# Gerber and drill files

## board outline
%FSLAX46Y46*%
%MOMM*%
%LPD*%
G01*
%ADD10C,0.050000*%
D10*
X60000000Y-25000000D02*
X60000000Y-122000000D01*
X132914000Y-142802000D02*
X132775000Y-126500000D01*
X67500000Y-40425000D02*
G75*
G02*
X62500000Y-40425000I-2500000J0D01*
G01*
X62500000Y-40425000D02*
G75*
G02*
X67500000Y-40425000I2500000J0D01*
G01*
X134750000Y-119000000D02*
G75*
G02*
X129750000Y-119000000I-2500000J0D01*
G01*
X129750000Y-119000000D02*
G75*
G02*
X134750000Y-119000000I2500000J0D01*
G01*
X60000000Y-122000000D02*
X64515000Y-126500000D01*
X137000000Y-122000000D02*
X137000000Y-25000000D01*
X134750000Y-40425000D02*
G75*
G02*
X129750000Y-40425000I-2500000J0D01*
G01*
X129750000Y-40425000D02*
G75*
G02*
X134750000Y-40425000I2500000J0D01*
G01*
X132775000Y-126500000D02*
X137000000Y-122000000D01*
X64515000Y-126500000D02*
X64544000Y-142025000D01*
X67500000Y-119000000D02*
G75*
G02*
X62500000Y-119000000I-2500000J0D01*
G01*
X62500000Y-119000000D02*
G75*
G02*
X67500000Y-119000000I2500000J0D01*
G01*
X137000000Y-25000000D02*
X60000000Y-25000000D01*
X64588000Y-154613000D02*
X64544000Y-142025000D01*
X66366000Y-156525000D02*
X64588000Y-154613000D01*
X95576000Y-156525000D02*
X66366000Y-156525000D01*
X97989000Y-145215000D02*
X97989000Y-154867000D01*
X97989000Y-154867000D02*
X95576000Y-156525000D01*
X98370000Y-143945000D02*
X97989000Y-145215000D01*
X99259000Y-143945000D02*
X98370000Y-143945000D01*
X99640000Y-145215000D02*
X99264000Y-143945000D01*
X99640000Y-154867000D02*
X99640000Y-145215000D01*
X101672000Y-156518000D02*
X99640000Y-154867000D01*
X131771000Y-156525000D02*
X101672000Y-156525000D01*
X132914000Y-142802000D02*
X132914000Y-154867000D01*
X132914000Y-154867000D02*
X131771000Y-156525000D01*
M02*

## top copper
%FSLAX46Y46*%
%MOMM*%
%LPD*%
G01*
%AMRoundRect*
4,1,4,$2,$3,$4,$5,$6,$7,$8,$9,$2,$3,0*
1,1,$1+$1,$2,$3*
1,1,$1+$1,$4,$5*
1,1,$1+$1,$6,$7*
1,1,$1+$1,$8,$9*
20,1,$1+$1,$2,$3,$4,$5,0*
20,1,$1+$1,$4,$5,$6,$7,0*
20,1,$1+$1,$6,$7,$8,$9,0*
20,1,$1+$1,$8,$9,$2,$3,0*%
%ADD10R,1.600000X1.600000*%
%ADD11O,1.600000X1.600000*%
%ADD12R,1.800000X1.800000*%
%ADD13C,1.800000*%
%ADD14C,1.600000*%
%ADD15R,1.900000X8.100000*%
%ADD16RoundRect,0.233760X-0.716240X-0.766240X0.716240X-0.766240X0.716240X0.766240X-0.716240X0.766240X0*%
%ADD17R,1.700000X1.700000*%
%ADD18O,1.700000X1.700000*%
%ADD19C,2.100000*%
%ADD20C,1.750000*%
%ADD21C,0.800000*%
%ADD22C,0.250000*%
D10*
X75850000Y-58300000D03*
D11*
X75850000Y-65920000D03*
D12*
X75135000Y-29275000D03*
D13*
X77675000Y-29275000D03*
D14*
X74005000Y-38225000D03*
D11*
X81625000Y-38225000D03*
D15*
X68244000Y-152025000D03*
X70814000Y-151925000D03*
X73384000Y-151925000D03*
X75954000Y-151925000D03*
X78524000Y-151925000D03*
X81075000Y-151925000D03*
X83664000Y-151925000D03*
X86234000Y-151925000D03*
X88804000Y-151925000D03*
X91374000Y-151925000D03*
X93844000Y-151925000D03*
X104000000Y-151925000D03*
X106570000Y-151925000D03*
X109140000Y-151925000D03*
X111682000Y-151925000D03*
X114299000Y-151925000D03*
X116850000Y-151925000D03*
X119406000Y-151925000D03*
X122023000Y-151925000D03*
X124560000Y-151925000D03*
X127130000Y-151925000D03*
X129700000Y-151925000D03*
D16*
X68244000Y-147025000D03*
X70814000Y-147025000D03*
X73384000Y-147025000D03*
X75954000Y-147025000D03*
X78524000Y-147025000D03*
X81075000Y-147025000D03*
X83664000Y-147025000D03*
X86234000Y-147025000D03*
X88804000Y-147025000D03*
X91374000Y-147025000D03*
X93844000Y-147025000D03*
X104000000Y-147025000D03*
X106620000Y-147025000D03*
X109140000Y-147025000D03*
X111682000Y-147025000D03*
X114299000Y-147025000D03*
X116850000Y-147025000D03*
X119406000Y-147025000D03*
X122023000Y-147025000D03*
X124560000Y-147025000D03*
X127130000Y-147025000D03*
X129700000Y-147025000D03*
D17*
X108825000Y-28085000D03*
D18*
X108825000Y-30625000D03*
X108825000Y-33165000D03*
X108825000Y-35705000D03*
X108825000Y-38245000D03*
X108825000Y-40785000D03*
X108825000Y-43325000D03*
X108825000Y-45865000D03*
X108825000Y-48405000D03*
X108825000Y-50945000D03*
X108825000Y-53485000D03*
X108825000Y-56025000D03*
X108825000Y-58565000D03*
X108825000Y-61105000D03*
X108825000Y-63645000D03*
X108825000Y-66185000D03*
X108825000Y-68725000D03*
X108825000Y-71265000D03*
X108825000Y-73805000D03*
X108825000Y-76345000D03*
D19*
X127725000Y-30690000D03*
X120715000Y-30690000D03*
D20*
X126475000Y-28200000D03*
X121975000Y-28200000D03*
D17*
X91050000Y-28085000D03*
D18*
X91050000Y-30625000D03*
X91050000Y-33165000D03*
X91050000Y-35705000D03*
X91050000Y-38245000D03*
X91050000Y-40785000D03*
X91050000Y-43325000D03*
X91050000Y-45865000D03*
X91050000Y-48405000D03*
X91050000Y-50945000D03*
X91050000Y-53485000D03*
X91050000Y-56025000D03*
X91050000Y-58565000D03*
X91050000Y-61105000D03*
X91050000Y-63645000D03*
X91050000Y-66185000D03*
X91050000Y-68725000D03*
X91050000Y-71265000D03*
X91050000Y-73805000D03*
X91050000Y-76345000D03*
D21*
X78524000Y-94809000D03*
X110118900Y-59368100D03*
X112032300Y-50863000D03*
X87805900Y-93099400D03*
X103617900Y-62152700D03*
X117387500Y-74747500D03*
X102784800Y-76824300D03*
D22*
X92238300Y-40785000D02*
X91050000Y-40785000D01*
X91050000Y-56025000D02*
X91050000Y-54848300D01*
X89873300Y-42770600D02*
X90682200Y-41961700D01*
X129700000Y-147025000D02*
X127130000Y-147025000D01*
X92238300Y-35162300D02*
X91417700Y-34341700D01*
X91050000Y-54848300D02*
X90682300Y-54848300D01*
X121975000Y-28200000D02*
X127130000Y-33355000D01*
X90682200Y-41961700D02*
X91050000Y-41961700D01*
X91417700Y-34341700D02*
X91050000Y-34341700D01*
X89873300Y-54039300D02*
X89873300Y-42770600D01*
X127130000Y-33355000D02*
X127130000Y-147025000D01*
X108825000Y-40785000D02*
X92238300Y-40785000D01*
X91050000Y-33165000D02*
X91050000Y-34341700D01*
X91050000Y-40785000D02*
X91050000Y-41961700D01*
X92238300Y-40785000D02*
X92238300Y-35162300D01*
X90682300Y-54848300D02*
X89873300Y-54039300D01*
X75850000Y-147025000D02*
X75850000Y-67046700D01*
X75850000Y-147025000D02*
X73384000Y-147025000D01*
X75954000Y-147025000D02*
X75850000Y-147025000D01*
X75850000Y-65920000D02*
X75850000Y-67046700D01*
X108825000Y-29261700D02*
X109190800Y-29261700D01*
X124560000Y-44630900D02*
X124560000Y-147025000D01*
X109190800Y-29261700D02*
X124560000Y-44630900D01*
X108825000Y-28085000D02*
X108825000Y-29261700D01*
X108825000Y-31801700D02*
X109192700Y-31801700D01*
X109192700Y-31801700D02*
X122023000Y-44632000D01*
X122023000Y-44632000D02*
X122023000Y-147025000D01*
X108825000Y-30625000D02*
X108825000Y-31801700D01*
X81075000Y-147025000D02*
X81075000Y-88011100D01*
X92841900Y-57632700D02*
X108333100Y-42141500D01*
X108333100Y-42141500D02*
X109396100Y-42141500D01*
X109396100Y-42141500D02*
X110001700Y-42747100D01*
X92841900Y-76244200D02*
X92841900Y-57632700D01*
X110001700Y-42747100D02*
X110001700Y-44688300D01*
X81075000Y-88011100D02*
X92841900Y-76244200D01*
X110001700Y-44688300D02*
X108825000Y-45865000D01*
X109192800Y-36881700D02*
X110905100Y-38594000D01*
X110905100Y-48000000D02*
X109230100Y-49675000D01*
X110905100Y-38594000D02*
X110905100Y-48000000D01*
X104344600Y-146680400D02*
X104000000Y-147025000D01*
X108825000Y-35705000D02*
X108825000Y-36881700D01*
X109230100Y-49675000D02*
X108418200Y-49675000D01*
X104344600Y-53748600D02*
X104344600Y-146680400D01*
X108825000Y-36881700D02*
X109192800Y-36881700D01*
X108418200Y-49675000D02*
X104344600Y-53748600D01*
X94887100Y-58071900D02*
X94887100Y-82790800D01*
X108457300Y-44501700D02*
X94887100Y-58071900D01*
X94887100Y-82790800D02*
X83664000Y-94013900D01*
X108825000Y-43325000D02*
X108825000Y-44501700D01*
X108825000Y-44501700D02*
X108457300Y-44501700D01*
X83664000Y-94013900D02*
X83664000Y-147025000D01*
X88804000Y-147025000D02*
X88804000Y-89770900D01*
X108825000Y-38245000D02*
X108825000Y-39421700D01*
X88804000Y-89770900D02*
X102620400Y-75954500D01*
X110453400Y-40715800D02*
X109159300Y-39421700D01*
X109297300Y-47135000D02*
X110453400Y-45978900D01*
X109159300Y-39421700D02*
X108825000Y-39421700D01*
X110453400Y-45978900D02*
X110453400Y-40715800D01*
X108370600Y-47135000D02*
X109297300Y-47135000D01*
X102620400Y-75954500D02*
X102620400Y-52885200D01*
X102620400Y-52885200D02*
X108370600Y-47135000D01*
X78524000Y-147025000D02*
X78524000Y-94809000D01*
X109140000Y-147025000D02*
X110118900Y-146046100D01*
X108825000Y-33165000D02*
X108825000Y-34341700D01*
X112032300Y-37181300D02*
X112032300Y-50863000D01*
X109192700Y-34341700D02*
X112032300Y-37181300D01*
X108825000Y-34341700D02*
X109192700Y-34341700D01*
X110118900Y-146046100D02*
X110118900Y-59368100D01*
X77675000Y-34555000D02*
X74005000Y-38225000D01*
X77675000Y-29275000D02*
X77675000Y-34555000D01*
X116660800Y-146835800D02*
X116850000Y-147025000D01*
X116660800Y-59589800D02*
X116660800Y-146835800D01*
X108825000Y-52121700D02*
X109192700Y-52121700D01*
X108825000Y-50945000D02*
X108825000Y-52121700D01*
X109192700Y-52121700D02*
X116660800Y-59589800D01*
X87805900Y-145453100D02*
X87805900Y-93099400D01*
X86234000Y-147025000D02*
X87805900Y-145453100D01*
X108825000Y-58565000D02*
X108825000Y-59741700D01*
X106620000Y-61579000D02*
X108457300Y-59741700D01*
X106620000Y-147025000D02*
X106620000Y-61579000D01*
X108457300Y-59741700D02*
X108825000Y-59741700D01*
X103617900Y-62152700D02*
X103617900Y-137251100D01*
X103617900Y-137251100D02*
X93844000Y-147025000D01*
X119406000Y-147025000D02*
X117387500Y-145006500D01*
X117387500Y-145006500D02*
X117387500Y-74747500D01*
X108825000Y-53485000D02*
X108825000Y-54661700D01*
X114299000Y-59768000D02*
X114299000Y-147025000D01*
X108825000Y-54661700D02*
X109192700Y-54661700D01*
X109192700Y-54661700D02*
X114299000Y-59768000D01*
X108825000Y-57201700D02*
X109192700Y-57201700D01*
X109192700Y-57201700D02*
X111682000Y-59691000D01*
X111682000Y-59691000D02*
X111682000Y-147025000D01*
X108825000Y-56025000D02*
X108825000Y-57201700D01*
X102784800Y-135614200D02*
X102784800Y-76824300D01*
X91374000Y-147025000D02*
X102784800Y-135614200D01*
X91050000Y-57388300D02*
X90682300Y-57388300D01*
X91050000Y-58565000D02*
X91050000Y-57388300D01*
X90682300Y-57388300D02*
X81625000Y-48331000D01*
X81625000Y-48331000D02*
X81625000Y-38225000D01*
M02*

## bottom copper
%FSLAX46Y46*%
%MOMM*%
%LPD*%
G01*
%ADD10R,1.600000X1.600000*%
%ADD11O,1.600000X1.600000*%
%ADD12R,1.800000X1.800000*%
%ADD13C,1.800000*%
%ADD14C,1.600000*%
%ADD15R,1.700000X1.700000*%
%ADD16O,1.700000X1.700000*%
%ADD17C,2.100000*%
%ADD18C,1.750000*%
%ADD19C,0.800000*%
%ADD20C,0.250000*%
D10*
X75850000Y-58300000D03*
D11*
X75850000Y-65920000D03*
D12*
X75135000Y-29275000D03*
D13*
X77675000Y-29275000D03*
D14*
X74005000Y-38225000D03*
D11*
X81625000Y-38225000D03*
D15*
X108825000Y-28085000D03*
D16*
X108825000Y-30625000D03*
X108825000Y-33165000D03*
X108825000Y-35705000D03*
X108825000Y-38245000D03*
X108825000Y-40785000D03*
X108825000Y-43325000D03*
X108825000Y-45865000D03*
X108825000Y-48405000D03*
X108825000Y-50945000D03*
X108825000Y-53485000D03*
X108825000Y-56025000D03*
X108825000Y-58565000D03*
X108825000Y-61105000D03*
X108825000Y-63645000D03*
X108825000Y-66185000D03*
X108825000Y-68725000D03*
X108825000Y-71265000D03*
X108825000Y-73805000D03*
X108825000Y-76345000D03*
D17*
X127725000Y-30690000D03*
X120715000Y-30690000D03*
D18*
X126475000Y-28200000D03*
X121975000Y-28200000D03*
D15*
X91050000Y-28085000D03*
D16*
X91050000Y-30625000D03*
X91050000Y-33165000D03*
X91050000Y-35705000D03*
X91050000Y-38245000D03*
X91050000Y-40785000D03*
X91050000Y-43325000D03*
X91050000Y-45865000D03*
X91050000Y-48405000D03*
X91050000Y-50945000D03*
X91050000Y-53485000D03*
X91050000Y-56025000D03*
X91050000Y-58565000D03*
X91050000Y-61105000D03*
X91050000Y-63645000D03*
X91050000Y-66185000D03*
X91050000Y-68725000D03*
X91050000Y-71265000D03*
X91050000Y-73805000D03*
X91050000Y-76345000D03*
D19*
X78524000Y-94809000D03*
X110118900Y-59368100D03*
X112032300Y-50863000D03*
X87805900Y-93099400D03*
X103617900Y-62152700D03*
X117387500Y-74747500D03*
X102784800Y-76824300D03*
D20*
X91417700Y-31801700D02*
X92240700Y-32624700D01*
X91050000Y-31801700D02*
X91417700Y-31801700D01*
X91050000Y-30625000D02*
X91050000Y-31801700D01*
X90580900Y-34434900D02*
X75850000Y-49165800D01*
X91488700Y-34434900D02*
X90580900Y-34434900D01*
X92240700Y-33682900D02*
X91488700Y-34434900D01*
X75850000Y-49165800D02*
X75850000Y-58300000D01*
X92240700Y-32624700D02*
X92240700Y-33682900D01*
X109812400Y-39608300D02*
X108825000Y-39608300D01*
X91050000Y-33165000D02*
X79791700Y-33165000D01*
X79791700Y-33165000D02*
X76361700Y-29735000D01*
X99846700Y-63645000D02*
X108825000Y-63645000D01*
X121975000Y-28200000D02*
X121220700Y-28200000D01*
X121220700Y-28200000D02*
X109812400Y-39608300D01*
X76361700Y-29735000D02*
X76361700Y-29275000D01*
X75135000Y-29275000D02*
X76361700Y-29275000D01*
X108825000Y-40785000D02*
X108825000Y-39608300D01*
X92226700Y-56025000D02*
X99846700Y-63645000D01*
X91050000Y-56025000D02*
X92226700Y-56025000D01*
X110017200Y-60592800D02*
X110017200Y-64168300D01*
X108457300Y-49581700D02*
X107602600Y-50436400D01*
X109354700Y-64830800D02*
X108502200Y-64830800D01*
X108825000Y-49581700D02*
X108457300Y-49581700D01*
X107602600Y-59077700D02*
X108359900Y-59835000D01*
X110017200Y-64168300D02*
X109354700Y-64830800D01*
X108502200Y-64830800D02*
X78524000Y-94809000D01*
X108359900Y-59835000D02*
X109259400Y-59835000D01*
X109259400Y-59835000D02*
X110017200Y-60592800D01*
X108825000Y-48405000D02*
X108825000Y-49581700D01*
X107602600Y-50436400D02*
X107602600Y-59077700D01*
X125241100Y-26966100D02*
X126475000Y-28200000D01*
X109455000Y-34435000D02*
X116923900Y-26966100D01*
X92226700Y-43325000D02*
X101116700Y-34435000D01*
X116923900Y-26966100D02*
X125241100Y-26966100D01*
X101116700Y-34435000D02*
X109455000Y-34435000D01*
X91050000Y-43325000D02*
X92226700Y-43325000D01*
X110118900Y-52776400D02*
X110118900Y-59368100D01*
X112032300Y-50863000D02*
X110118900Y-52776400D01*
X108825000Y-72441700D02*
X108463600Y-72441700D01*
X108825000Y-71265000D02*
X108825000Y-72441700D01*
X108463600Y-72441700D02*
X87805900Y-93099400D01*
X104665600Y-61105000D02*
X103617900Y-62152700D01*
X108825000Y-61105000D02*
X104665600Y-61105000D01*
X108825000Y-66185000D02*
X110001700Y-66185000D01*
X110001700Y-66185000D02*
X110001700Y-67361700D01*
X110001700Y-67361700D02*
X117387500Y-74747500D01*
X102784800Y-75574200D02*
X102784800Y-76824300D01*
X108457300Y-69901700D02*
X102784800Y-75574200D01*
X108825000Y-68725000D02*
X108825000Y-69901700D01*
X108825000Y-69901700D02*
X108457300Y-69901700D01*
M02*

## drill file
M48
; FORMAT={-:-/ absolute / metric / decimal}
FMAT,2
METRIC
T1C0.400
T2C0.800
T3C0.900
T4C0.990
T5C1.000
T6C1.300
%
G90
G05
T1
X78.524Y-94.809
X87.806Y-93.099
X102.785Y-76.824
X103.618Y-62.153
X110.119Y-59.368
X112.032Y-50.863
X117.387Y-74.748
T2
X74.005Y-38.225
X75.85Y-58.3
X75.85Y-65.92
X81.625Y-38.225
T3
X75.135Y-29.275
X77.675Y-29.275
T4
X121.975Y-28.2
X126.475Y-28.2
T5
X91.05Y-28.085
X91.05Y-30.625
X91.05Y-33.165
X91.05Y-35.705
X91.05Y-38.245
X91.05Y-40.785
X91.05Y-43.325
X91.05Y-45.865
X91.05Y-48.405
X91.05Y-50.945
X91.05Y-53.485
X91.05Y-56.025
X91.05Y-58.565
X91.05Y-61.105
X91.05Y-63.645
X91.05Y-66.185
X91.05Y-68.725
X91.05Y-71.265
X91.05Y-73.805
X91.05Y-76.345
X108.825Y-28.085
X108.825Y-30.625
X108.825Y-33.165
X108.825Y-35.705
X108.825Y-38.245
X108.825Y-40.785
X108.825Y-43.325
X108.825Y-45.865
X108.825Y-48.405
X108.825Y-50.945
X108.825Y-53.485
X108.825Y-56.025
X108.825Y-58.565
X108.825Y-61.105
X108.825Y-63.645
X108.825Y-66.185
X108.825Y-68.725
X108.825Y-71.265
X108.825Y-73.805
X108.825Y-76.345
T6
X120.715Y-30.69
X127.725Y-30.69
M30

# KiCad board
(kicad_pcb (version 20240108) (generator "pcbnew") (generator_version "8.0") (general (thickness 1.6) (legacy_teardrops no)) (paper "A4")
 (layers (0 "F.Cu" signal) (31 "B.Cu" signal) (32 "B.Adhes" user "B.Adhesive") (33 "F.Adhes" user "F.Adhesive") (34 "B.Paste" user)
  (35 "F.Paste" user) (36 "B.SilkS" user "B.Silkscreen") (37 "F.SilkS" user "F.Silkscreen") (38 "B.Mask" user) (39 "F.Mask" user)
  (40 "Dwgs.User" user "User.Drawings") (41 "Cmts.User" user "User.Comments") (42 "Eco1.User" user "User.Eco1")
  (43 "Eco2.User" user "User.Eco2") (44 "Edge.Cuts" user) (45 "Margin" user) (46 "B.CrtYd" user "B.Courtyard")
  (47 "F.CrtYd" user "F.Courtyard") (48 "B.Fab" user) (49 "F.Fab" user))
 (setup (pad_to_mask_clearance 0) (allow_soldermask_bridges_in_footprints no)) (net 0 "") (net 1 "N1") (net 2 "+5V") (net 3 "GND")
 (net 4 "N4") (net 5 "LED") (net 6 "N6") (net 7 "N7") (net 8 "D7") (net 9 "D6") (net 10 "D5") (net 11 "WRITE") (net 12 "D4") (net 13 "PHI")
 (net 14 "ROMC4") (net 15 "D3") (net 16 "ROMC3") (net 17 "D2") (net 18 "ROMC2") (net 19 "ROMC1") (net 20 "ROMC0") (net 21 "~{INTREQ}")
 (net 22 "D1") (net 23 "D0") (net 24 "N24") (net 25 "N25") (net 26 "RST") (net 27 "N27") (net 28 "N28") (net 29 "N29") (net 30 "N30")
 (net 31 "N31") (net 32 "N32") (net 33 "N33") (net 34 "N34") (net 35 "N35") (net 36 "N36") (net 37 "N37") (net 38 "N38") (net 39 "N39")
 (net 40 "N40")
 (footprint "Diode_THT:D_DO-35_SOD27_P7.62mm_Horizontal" (layer "F.Cu") (at 75.85 58.3 -90)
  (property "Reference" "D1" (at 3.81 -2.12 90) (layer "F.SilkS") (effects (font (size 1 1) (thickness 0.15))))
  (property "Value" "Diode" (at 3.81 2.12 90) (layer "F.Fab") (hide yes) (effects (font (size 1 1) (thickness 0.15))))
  (pad "1" thru_hole rect (at 0 0 270) (size 1.6 1.6) (drill 0.8) (layers "*.Cu" "*.Mask") (remove_unused_layers no) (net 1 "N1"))
  (pad "2" thru_hole oval (at 7.62 0 270) (size 1.6 1.6) (drill 0.8) (layers "*.Cu" "*.Mask") (remove_unused_layers no) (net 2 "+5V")))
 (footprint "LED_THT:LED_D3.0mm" (layer "F.Cu") (at 75.135 29.275)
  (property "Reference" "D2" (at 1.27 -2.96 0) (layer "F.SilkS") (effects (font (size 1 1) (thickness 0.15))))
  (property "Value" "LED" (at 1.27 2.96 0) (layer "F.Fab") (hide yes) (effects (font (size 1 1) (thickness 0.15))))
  (pad "1" thru_hole rect (at 0 0) (size 1.8 1.8) (drill 0.9) (layers "*.Cu" "*.Mask") (remove_unused_layers no) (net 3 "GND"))
  (pad "2" thru_hole circle (at 2.54 0) (size 1.8 1.8) (drill 0.9) (layers "*.Cu" "*.Mask") (remove_unused_layers no) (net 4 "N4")))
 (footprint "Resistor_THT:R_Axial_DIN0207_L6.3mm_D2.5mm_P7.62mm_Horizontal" (layer "F.Cu") (at 74.005 38.225)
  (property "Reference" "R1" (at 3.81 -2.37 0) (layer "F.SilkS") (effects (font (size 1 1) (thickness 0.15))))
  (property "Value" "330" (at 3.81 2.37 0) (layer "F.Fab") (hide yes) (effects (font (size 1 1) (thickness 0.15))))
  (pad "1" thru_hole circle (at 0 0) (size 1.6 1.6) (drill 0.8) (layers "*.Cu" "*.Mask") (remove_unused_layers no) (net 4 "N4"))
  (pad "2" thru_hole oval (at 7.62 0) (size 1.6 1.6) (drill 0.8) (layers "*.Cu" "*.Mask") (remove_unused_layers no) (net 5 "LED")))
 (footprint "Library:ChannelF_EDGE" (layer "F.Cu") (at 68.144 149.025)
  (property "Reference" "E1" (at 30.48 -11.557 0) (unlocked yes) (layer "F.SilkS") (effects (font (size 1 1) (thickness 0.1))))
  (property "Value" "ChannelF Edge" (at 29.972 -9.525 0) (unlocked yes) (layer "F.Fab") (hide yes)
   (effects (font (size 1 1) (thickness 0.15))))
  (fp_line (start -3.556 5.588) (end -3.6 -7) (stroke (width 0.05) (type default)) (layer "Edge.Cuts"))
  (fp_line (start -1.778 7.5) (end -3.556 5.588) (stroke (width 0.05) (type default)) (layer "Edge.Cuts"))
  (fp_line (start 27.432 7.5) (end -1.778 7.5) (stroke (width 0.05) (type default)) (layer "Edge.Cuts"))
  (fp_line (start 29.845 -3.81) (end 29.845 5.842) (stroke (width 0.05) (type default)) (layer "Edge.Cuts"))
  (fp_line (start 29.845 5.842) (end 27.432 7.5) (stroke (width 0.05) (type default)) (layer "Edge.Cuts"))
  (fp_line (start 30.226 -5.08) (end 29.845 -3.81) (stroke (width 0.05) (type default)) (layer "Edge.Cuts"))
  (fp_line (start 31.115 -5.08) (end 30.226 -5.08) (stroke (width 0.05) (type default)) (layer "Edge.Cuts"))
  (fp_line (start 31.496 -3.81) (end 31.12 -5.08) (stroke (width 0.05) (type default)) (layer "Edge.Cuts"))
  (fp_line (start 31.496 5.842) (end 31.496 -3.81) (stroke (width 0.05) (type default)) (layer "Edge.Cuts"))
  (fp_line (start 33.528 7.493) (end 31.496 5.842) (stroke (width 0.05) (type default)) (layer "Edge.Cuts"))
  (fp_line (start 63.627 7.5) (end 33.528 7.5) (stroke (width 0.05) (type default)) (layer "Edge.Cuts"))
  (fp_line (start 64.77 -6.223) (end 64.77 5.842) (stroke (width 0.05) (type default)) (layer "Edge.Cuts"))
  (fp_line (start 64.77 5.842) (end 63.627 7.5) (stroke (width 0.05) (type default)) (layer "Edge.Cuts"))
  (pad "" smd rect (at 0.1 3) (size 1.9 8.1) (layers "F.Cu" "F.Paste" "F.Mask"))
  (pad "" smd rect (at 2.67 2.9) (size 1.9 8.1) (layers "F.Cu" "F.Paste" "F.Mask"))
  (pad "" smd rect (at 5.24 2.9) (size 1.9 8.1) (layers "F.Cu" "F.Paste" "F.Mask"))
  (pad "" smd rect (at 7.81 2.9) (size 1.9 8.1) (layers "F.Cu" "F.Paste" "F.Mask"))
  (pad "" smd rect (at 10.38 2.9) (size 1.9 8.1) (layers "F.Cu" "F.Paste" "F.Mask"))
  (pad "" smd rect (at 12.931 2.9) (size 1.9 8.1) (layers "F.Cu" "F.Paste" "F.Mask"))
  (pad "" smd rect (at 15.52 2.9) (size 1.9 8.1) (layers "F.Cu" "F.Paste" "F.Mask"))
  (pad "" smd rect (at 18.09 2.9) (size 1.9 8.1) (layers "F.Cu" "F.Paste" "F.Mask"))
  (pad "" smd rect (at 20.66 2.9) (size 1.9 8.1) (layers "F.Cu" "F.Paste" "F.Mask"))
  (pad "" smd rect (at 23.23 2.9) (size 1.9 8.1) (layers "F.Cu" "F.Paste" "F.Mask"))
  (pad "" smd rect (at 25.7 2.9) (size 1.9 8.1) (layers "F.Cu" "F.Paste" "F.Mask"))
  (pad "" smd rect (at 35.856 2.9) (size 1.9 8.1) (layers "F.Cu" "F.Paste" "F.Mask"))
  (pad "" smd rect (at 38.426 2.9) (size 1.9 8.1) (layers "F.Cu" "F.Paste" "F.Mask"))
  (pad "" smd rect (at 40.996 2.9) (size 1.9 8.1) (layers "F.Cu" "F.Paste" "F.Mask"))
  (pad "" smd rect (at 43.538 2.9) (size 1.9 8.1) (layers "F.Cu" "F.Paste" "F.Mask"))
  (pad "" smd rect (at 46.155 2.9) (size 1.9 8.1) (layers "F.Cu" "F.Paste" "F.Mask"))
  (pad "" smd rect (at 48.706 2.9) (size 1.9 8.1) (layers "F.Cu" "F.Paste" "F.Mask"))
  (pad "" smd rect (at 51.262 2.9) (size 1.9 8.1) (layers "F.Cu" "F.Paste" "F.Mask"))
  (pad "" smd rect (at 53.879 2.9) (size 1.9 8.1) (layers "F.Cu" "F.Paste" "F.Mask"))
  (pad "" smd rect (at 56.416 2.9) (size 1.9 8.1) (layers "F.Cu" "F.Paste" "F.Mask"))
  (pad "" smd rect (at 58.986 2.9) (size 1.9 8.1) (layers "F.Cu" "F.Paste" "F.Mask"))
  (pad "" smd rect (at 61.556 2.9) (size 1.9 8.1) (layers "F.Cu" "F.Paste" "F.Mask"))
  (pad "1" smd roundrect (at 0.1 -2) (size 1.9 2) (layers "F.Cu" "F.Paste" "F.Mask") (roundrect_rratio 0.1230314961) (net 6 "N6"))
  (pad "2" smd roundrect (at 2.67 -2) (size 1.9 2) (layers "F.Cu" "F.Paste" "F.Mask") (roundrect_rratio 0.1230314961) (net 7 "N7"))
  (pad "3" smd roundrect (at 5.24 -2) (size 1.9 2) (layers "F.Cu" "F.Paste" "F.Mask") (roundrect_rratio 0.1230314961) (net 2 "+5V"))
  (pad "4" smd roundrect (at 7.81 -2) (size 1.9 2) (layers "F.Cu" "F.Paste" "F.Mask") (roundrect_rratio 0.1230314961) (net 2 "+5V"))
  (pad "5" smd roundrect (at 10.38 -2) (size 1.9 2) (layers "F.Cu" "F.Paste" "F.Mask") (roundrect_rratio 0.1230314961) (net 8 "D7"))
  (pad "6" smd roundrect (at 12.931 -2) (size 1.9 2) (layers "F.Cu" "F.Paste" "F.Mask") (roundrect_rratio 0.1230314961) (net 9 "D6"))
  (pad "7" smd roundrect (at 15.52 -2) (size 1.9 2) (layers "F.Cu" "F.Paste" "F.Mask") (roundrect_rratio 0.1230314961) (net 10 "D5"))
  (pad "8" smd roundrect (at 18.09 -2) (size 1.9 2) (layers "F.Cu" "F.Paste" "F.Mask") (roundrect_rratio 0.1230314961) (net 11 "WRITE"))
  (pad "9" smd roundrect (at 20.66 -2) (size 1.9 2) (layers "F.Cu" "F.Paste" "F.Mask") (roundrect_rratio 0.1230314961) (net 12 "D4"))
  (pad "10" smd roundrect (at 23.23 -2) (size 1.9 2) (layers "F.Cu" "F.Paste" "F.Mask") (roundrect_rratio 0.1230314961) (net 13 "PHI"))
  (pad "11" smd roundrect (at 25.7 -2) (size 1.9 2) (layers "F.Cu" "F.Paste" "F.Mask") (roundrect_rratio 0.1230314961) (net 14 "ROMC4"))
  (pad "12" smd roundrect (at 35.856 -2) (size 1.9 2) (layers "F.Cu" "F.Paste" "F.Mask") (roundrect_rratio 0.1230314961) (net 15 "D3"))
  (pad "13" smd roundrect (at 38.476 -2) (size 1.9 2) (layers "F.Cu" "F.Paste" "F.Mask") (roundrect_rratio 0.1230314961) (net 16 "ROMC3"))
  (pad "14" smd roundrect (at 40.996 -2) (size 1.9 2) (layers "F.Cu" "F.Paste" "F.Mask") (roundrect_rratio 0.1230314961) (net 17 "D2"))
  (pad "15" smd roundrect (at 43.538 -2) (size 1.9 2) (layers "F.Cu" "F.Paste" "F.Mask") (roundrect_rratio 0.1230314961) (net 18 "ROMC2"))
  (pad "16" smd roundrect (at 46.155 -2) (size 1.9 2) (layers "F.Cu" "F.Paste" "F.Mask") (roundrect_rratio 0.1230314961) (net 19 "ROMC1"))
  (pad "17" smd roundrect (at 48.706 -2) (size 1.9 2) (layers "F.Cu" "F.Paste" "F.Mask") (roundrect_rratio 0.1230314961) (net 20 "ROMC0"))
  (pad "18" smd roundrect (at 51.262 -2) (size 1.9 2) (layers "F.Cu" "F.Paste" "F.Mask") (roundrect_rratio 0.1230314961)
   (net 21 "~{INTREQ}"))
  (pad "19" smd roundrect (at 53.879 -2) (size 1.9 2) (layers "F.Cu" "F.Paste" "F.Mask") (roundrect_rratio 0.1230314961) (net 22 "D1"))
  (pad "20" smd roundrect (at 56.416 -2) (size 1.9 2) (layers "F.Cu" "F.Paste" "F.Mask") (roundrect_rratio 0.1230314961) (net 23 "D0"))
  (pad "21" smd roundrect (at 58.986 -2) (size 1.9 2) (layers "F.Cu" "F.Paste" "F.Mask") (roundrect_rratio 0.1230314961) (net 3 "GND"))
  (pad "22" smd roundrect (at 61.556 -2) (size 1.9 2) (layers "F.Cu" "F.Paste" "F.Mask") (roundrect_rratio 0.1230314961) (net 3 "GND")))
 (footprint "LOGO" (layer "B.Cu") (at 97.683578 89.128118 180)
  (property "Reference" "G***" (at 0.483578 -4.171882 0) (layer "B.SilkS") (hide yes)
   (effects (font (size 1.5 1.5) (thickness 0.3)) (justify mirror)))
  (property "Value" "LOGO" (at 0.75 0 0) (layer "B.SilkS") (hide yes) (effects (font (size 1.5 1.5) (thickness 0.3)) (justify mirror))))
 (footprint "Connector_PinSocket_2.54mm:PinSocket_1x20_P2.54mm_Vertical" (layer "B.Cu") (at 108.825 28.085 180)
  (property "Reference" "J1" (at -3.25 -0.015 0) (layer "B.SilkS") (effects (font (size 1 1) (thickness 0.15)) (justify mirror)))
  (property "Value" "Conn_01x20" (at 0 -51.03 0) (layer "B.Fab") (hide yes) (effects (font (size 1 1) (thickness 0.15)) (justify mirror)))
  (pad "1" thru_hole rect (at 0 0 180) (size 1.7 1.7) (drill 1) (layers "*.Cu" "*.Mask") (remove_unused_layers no) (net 23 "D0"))
  (pad "2" thru_hole oval (at 0 -2.54 180) (size 1.7 1.7) (drill 1) (layers "*.Cu" "*.Mask") (remove_unused_layers no) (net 22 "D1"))
  (pad "3" thru_hole oval (at 0 -5.08 180) (size 1.7 1.7) (drill 1) (layers "*.Cu" "*.Mask") (remove_unused_layers no) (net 17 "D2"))
  (pad "4" thru_hole oval (at 0 -7.62 180) (size 1.7 1.7) (drill 1) (layers "*.Cu" "*.Mask") (remove_unused_layers no) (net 15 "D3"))
  (pad "5" thru_hole oval (at 0 -10.16 180) (size 1.7 1.7) (drill 1) (layers "*.Cu" "*.Mask") (remove_unused_layers no) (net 12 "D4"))
  (pad "6" thru_hole oval (at 0 -12.7 180) (size 1.7 1.7) (drill 1) (layers "*.Cu" "*.Mask") (remove_unused_layers no) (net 3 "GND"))
  (pad "7" thru_hole oval (at 0 -15.24 180) (size 1.7 1.7) (drill 1) (layers "*.Cu" "*.Mask") (remove_unused_layers no) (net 10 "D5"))
  (pad "8" thru_hole oval (at 0 -17.78 180) (size 1.7 1.7) (drill 1) (layers "*.Cu" "*.Mask") (remove_unused_layers no) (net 9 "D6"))
  (pad "9" thru_hole oval (at 0 -20.32 180) (size 1.7 1.7) (drill 1) (layers "*.Cu" "*.Mask") (remove_unused_layers no) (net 8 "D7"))
  (pad "10" thru_hole oval (at 0 -22.86 180) (size 1.7 1.7) (drill 1) (layers "*.Cu" "*.Mask") (remove_unused_layers no) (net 20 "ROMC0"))
  (pad "11" thru_hole oval (at 0 -25.4 180) (size 1.7 1.7) (drill 1) (layers "*.Cu" "*.Mask") (remove_unused_layers no) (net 19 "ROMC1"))
  (pad "12" thru_hole oval (at 0 -27.94 180) (size 1.7 1.7) (drill 1) (layers "*.Cu" "*.Mask") (remove_unused_layers no) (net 18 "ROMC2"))
  (pad "13" thru_hole oval (at 0 -30.48 180) (size 1.7 1.7) (drill 1) (layers "*.Cu" "*.Mask") (remove_unused_layers no) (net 16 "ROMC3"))
  (pad "14" thru_hole oval (at 0 -33.02 180) (size 1.7 1.7) (drill 1) (layers "*.Cu" "*.Mask") (remove_unused_layers no) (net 14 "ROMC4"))
  (pad "15" thru_hole oval (at 0 -35.56 180) (size 1.7 1.7) (drill 1) (layers "*.Cu" "*.Mask") (remove_unused_layers no) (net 3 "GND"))
  (pad "16" thru_hole oval (at 0 -38.1 180) (size 1.7 1.7) (drill 1) (layers "*.Cu" "*.Mask") (remove_unused_layers no) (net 21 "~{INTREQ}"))
  (pad "17" thru_hole oval (at 0 -40.64 180) (size 1.7 1.7) (drill 1) (layers "*.Cu" "*.Mask") (remove_unused_layers no) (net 13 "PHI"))
  (pad "18" thru_hole oval (at 0 -43.18 180) (size 1.7 1.7) (drill 1) (layers "*.Cu" "*.Mask") (remove_unused_layers no) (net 11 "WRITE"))
  (pad "19" thru_hole oval (at 0 -45.72 180) (size 1.7 1.7) (drill 1) (layers "*.Cu" "*.Mask") (remove_unused_layers no) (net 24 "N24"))
  (pad "20" thru_hole oval (at 0 -48.26 180) (size 1.7 1.7) (drill 1) (layers "*.Cu" "*.Mask") (remove_unused_layers no) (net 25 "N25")))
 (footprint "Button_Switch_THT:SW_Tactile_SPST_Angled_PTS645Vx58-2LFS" (layer "B.Cu") (at 126.475 28.2 180)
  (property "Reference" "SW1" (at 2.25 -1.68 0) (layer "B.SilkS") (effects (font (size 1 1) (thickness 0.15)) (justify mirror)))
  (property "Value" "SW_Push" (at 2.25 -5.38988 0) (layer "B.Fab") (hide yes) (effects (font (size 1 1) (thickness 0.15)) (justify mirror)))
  (pad "" thru_hole circle (at -1.25 -2.49 180) (size 2.1 2.1) (drill 1.3) (layers "*.Cu" "*.Mask") (remove_unused_layers no))
  (pad "" thru_hole circle (at 5.76 -2.49 180) (size 2.1 2.1) (drill 1.3) (layers "*.Cu" "*.Mask") (remove_unused_layers no))
  (pad "1" thru_hole circle (at 0 0 180) (size 1.75 1.75) (drill 0.99) (layers "*.Cu" "*.Mask") (remove_unused_layers no) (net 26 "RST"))
  (pad "2" thru_hole circle (at 4.5 0 180) (size 1.75 1.75) (drill 0.99) (layers "*.Cu" "*.Mask") (remove_unused_layers no) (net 3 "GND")))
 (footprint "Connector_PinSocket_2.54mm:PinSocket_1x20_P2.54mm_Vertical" (layer "B.Cu") (at 91.05 28.085 180)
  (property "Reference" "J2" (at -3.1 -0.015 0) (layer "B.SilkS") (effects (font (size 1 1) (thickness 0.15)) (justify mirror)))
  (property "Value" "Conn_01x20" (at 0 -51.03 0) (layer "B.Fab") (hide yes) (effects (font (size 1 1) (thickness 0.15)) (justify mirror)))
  (pad "1" thru_hole rect (at 0 0 180) (size 1.7 1.7) (drill 1) (layers "*.Cu" "*.Mask") (remove_unused_layers no) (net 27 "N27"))
  (pad "2" thru_hole oval (at 0 -2.54 180) (size 1.7 1.7) (drill 1) (layers "*.Cu" "*.Mask") (remove_unused_layers no) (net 1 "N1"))
  (pad "3" thru_hole oval (at 0 -5.08 180) (size 1.7 1.7) (drill 1) (layers "*.Cu" "*.Mask") (remove_unused_layers no) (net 3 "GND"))
  (pad "4" thru_hole oval (at 0 -7.62 180) (size 1.7 1.7) (drill 1) (layers "*.Cu" "*.Mask") (remove_unused_layers no) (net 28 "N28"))
  (pad "5" thru_hole oval (at 0 -10.16 180) (size 1.7 1.7) (drill 1) (layers "*.Cu" "*.Mask") (remove_unused_layers no) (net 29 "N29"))
  (pad "6" thru_hole oval (at 0 -12.7 180) (size 1.7 1.7) (drill 1) (layers "*.Cu" "*.Mask") (remove_unused_layers no) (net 3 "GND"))
  (pad "7" thru_hole oval (at 0 -15.24 180) (size 1.7 1.7) (drill 1) (layers "*.Cu" "*.Mask") (remove_unused_layers no) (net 26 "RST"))
  (pad "8" thru_hole oval (at 0 -17.78 180) (size 1.7 1.7) (drill 1) (layers "*.Cu" "*.Mask") (remove_unused_layers no) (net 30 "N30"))
  (pad "9" thru_hole oval (at 0 -20.32 180) (size 1.7 1.7) (drill 1) (layers "*.Cu" "*.Mask") (remove_unused_layers no) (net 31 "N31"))
  (pad "10" thru_hole oval (at 0 -22.86 180) (size 1.7 1.7) (drill 1) (layers "*.Cu" "*.Mask") (remove_unused_layers no) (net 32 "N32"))
  (pad "11" thru_hole oval (at 0 -25.4 180) (size 1.7 1.7) (drill 1) (layers "*.Cu" "*.Mask") (remove_unused_layers no) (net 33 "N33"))
  (pad "12" thru_hole oval (at 0 -27.94 180) (size 1.7 1.7) (drill 1) (layers "*.Cu" "*.Mask") (remove_unused_layers no) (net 3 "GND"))
  (pad "13" thru_hole oval (at 0 -30.48 180) (size 1.7 1.7) (drill 1) (layers "*.Cu" "*.Mask") (remove_unused_layers no) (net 5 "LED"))
  (pad "14" thru_hole oval (at 0 -33.02 180) (size 1.7 1.7) (drill 1) (layers "*.Cu" "*.Mask") (remove_unused_layers no) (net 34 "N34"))
  (pad "15" thru_hole oval (at 0 -35.56 180) (size 1.7 1.7) (drill 1) (layers "*.Cu" "*.Mask") (remove_unused_layers no) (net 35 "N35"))
  (pad "16" thru_hole oval (at 0 -38.1 180) (size 1.7 1.7) (drill 1) (layers "*.Cu" "*.Mask") (remove_unused_layers no) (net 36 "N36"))
  (pad "17" thru_hole oval (at 0 -40.64 180) (size 1.7 1.7) (drill 1) (layers "*.Cu" "*.Mask") (remove_unused_layers no) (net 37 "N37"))
  (pad "18" thru_hole oval (at 0 -43.18 180) (size 1.7 1.7) (drill 1) (layers "*.Cu" "*.Mask") (remove_unused_layers no) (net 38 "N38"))
  (pad "19" thru_hole oval (at 0 -45.72 180) (size 1.7 1.7) (drill 1) (layers "*.Cu" "*.Mask") (remove_unused_layers no) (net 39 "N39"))
  (pad "20" thru_hole oval (at 0 -48.26 180) (size 1.7 1.7) (drill 1) (layers "*.Cu" "*.Mask") (remove_unused_layers no) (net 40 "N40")))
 (gr_line (start 60 25) (end 60 122) (stroke (width 0.05) (type default)) (layer "Edge.Cuts"))
 (gr_line (start 132.914 142.802) (end 132.775 126.5) (stroke (width 0.05) (type default)) (layer "Edge.Cuts"))
 (gr_circle (center 65 40.425) (end 67.5 40.425) (stroke (width 0.05) (type default)) (fill none) (layer "Edge.Cuts"))
 (gr_circle (center 132.25 119) (end 134.75 119) (stroke (width 0.05) (type default)) (fill none) (layer "Edge.Cuts"))
 (gr_line (start 60 122) (end 64.515 126.5) (stroke (width 0.05) (type default)) (layer "Edge.Cuts"))
 (gr_line (start 137 122) (end 137 25) (stroke (width 0.05) (type default)) (layer "Edge.Cuts"))
 (gr_circle (center 132.25 40.425) (end 134.75 40.425) (stroke (width 0.05) (type default)) (fill none) (layer "Edge.Cuts"))
 (gr_line (start 132.775 126.5) (end 137 122) (stroke (width 0.05) (type default)) (layer "Edge.Cuts"))
 (gr_line (start 64.515 126.5) (end 64.544 142.025) (stroke (width 0.05) (type default)) (layer "Edge.Cuts"))
 (gr_circle (center 65 119) (end 67.5 119) (stroke (width 0.05) (type default)) (fill none) (layer "Edge.Cuts"))
 (gr_line (start 137 25) (end 60 25) (stroke (width 0.05) (type default)) (layer "Edge.Cuts"))
 (segment (start 91.4177 31.8017) (end 92.2407 32.6247) (width 0.25) (layer "B.Cu") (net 1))
 (segment (start 91.05 31.8017) (end 91.4177 31.8017) (width 0.25) (layer "B.Cu") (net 1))
 (segment (start 91.05 30.625) (end 91.05 31.8017) (width 0.25) (layer "B.Cu") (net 1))
 (segment (start 90.5809 34.4349) (end 75.85 49.1658) (width 0.25) (layer "B.Cu") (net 1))
 (segment (start 91.4887 34.4349) (end 90.5809 34.4349) (width 0.25) (layer "B.Cu") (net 1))
 (segment (start 92.2407 33.6829) (end 91.4887 34.4349) (width 0.25) (layer "B.Cu") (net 1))
 (segment (start 75.85 49.1658) (end 75.85 58.3) (width 0.25) (layer "B.Cu") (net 1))
 (segment (start 92.2407 32.6247) (end 92.2407 33.6829) (width 0.25) (layer "B.Cu") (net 1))
 (segment (start 92.2383 40.785) (end 91.05 40.785) (width 0.25) (layer "F.Cu") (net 3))
 (segment (start 91.05 56.025) (end 91.05 54.8483) (width 0.25) (layer "F.Cu") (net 3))
 (segment (start 89.8733 42.7706) (end 90.6822 41.9617) (width 0.25) (layer "F.Cu") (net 3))
 (segment (start 129.7 147.025) (end 127.13 147.025) (width 0.25) (layer "F.Cu") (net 3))
 (segment (start 92.2383 35.1623) (end 91.4177 34.3417) (width 0.25) (layer "F.Cu") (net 3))
 (segment (start 91.05 54.8483) (end 90.6823 54.8483) (width 0.25) (layer "F.Cu") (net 3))
 (segment (start 121.975 28.2) (end 127.13 33.355) (width 0.25) (layer "F.Cu") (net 3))
 (segment (start 90.6822 41.9617) (end 91.05 41.9617) (width 0.25) (layer "F.Cu") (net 3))
 (segment (start 91.4177 34.3417) (end 91.05 34.3417) (width 0.25) (layer "F.Cu") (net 3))
 (segment (start 89.8733 54.0393) (end 89.8733 42.7706) (width 0.25) (layer "F.Cu") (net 3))
 (segment (start 127.13 33.355) (end 127.13 147.025) (width 0.25) (layer "F.Cu") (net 3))
 (segment (start 108.825 40.785) (end 92.2383 40.785) (width 0.25) (layer "F.Cu") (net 3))
 (segment (start 91.05 33.165) (end 91.05 34.3417) (width 0.25) (layer "F.Cu") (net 3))
 (segment (start 91.05 40.785) (end 91.05 41.9617) (width 0.25) (layer "F.Cu") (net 3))
 (segment (start 92.2383 40.785) (end 92.2383 35.1623) (width 0.25) (layer "F.Cu") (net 3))
 (segment (start 90.6823 54.8483) (end 89.8733 54.0393) (width 0.25) (layer "F.Cu") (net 3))
 (segment (start 109.8124 39.6083) (end 108.825 39.6083) (width 0.25) (layer "B.Cu") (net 3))
 (segment (start 91.05 33.165) (end 79.7917 33.165) (width 0.25) (layer "B.Cu") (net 3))
 (segment (start 79.7917 33.165) (end 76.3617 29.735) (width 0.25) (layer "B.Cu") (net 3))
 (segment (start 99.8467 63.645) (end 108.825 63.645) (width 0.25) (layer "B.Cu") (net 3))
 (segment (start 121.975 28.2) (end 121.2207 28.2) (width 0.25) (layer "B.Cu") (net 3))
 (segment (start 121.2207 28.2) (end 109.8124 39.6083) (width 0.25) (layer "B.Cu") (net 3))
 (segment (start 76.3617 29.735) (end 76.3617 29.275) (width 0.25) (layer "B.Cu") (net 3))
 (segment (start 75.135 29.275) (end 76.3617 29.275) (width 0.25) (layer "B.Cu") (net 3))
 (segment (start 108.825 40.785) (end 108.825 39.6083) (width 0.25) (layer "B.Cu") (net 3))
 (segment (start 92.2267 56.025) (end 99.8467 63.645) (width 0.25) (layer "B.Cu") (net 3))
 (segment (start 91.05 56.025) (end 92.2267 56.025) (width 0.25) (layer "B.Cu") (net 3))
 (segment (start 75.85 147.025) (end 75.85 67.0467) (width 0.25) (layer "F.Cu") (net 2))
 (segment (start 75.85 147.025) (end 73.384 147.025) (width 0.25) (layer "F.Cu") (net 2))
 (segment (start 75.954 147.025) (end 75.85 147.025) (width 0.25) (layer "F.Cu") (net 2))
 (segment (start 75.85 65.92) (end 75.85 67.0467) (width 0.25) (layer "F.Cu") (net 2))
 (segment (start 108.825 29.2617) (end 109.1908 29.2617) (width 0.25) (layer "F.Cu") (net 23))
 (segment (start 124.56 44.6309) (end 124.56 147.025) (width 0.25) (layer "F.Cu") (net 23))
 (segment (start 109.1908 29.2617) (end 124.56 44.6309) (width 0.25) (layer "F.Cu") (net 23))
 (segment (start 108.825 28.085) (end 108.825 29.2617) (width 0.25) (layer "F.Cu") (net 23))
 (segment (start 108.825 31.8017) (end 109.1927 31.8017) (width 0.25) (layer "F.Cu") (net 22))
 (segment (start 109.1927 31.8017) (end 122.023 44.632) (width 0.25) (layer "F.Cu") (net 22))
 (segment (start 122.023 44.632) (end 122.023 147.025) (width 0.25) (layer "F.Cu") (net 22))
 (segment (start 108.825 30.625) (end 108.825 31.8017) (width 0.25) (layer "F.Cu") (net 22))
 (segment (start 81.075 147.025) (end 81.075 88.0111) (width 0.25) (layer "F.Cu") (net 9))
 (segment (start 92.8419 57.6327) (end 108.3331 42.1415) (width 0.25) (layer "F.Cu") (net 9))
 (segment (start 108.3331 42.1415) (end 109.3961 42.1415) (width 0.25) (layer "F.Cu") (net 9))
 (segment (start 109.3961 42.1415) (end 110.0017 42.7471) (width 0.25) (layer "F.Cu") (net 9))
 (segment (start 92.8419 76.2442) (end 92.8419 57.6327) (width 0.25) (layer "F.Cu") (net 9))
 (segment (start 110.0017 42.7471) (end 110.0017 44.6883) (width 0.25) (layer "F.Cu") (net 9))
 (segment (start 81.075 88.0111) (end 92.8419 76.2442) (width 0.25) (layer "F.Cu") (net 9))
 (segment (start 110.0017 44.6883) (end 108.825 45.865) (width 0.25) (layer "F.Cu") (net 9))
 (segment (start 109.1928 36.8817) (end 110.9051 38.594) (width 0.25) (layer "F.Cu") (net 15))
 (segment (start 110.9051 48) (end 109.2301 49.675) (width 0.25) (layer "F.Cu") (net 15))
 (segment (start 110.9051 38.594) (end 110.9051 48) (width 0.25) (layer "F.Cu") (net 15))
 (segment (start 104.3446 146.6804) (end 104 147.025) (width 0.25) (layer "F.Cu") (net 15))
 (segment (start 108.825 35.705) (end 108.825 36.8817) (width 0.25) (layer "F.Cu") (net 15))
 (segment (start 109.2301 49.675) (end 108.4182 49.675) (width 0.25) (layer "F.Cu") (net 15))
 (segment (start 104.3446 53.7486) (end 104.3446 146.6804) (width 0.25) (layer "F.Cu") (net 15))
 (segment (start 108.825 36.8817) (end 109.1928 36.8817) (width 0.25) (layer "F.Cu") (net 15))
 (segment (start 108.4182 49.675) (end 104.3446 53.7486) (width 0.25) (layer "F.Cu") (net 15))
 (segment (start 94.8871 58.0719) (end 94.8871 82.7908) (width 0.25) (layer "F.Cu") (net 10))
 (segment (start 108.4573 44.5017) (end 94.8871 58.0719) (width 0.25) (layer "F.Cu") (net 10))
 (segment (start 94.8871 82.7908) (end 83.664 94.0139) (width 0.25) (layer "F.Cu") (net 10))
 (segment (start 108.825 43.325) (end 108.825 44.5017) (width 0.25) (layer "F.Cu") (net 10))
 (segment (start 108.825 44.5017) (end 108.4573 44.5017) (width 0.25) (layer "F.Cu") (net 10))
 (segment (start 83.664 94.0139) (end 83.664 147.025) (width 0.25) (layer "F.Cu") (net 10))
 (segment (start 88.804 147.025) (end 88.804 89.7709) (width 0.25) (layer "F.Cu") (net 12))
 (segment (start 108.825 38.245) (end 108.825 39.4217) (width 0.25) (layer "F.Cu") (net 12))
 (segment (start 88.804 89.7709) (end 102.6204 75.9545) (width 0.25) (layer "F.Cu") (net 12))
 (segment (start 110.4534 40.7158) (end 109.1593 39.4217) (width 0.25) (layer "F.Cu") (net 12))
 (segment (start 109.2973 47.135) (end 110.4534 45.9789) (width 0.25) (layer "F.Cu") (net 12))
 (segment (start 109.1593 39.4217) (end 108.825 39.4217) (width 0.25) (layer "F.Cu") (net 12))
 (segment (start 110.4534 45.9789) (end 110.4534 40.7158) (width 0.25) (layer "F.Cu") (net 12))
 (segment (start 108.3706 47.135) (end 109.2973 47.135) (width 0.25) (layer "F.Cu") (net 12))
 (segment (start 102.6204 75.9545) (end 102.6204 52.8852) (width 0.25) (layer "F.Cu") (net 12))
 (segment (start 102.6204 52.8852) (end 108.3706 47.135) (width 0.25) (layer "F.Cu") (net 12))
 (segment (start 78.524 147.025) (end 78.524 94.809) (width 0.25) (layer "F.Cu") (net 8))
 (via (at 78.524 94.809) (size 0.8) (drill 0.4) (layers "F.Cu" "B.Cu") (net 8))
 (segment (start 110.0172 60.5928) (end 110.0172 64.1683) (width 0.25) (layer "B.Cu") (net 8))
 (segment (start 108.4573 49.5817) (end 107.6026 50.4364) (width 0.25) (layer "B.Cu") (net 8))
 (segment (start 109.3547 64.8308) (end 108.5022 64.8308) (width 0.25) (layer "B.Cu") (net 8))
 (segment (start 108.825 49.5817) (end 108.4573 49.5817) (width 0.25) (layer "B.Cu") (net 8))
 (segment (start 107.6026 59.0777) (end 108.3599 59.835) (width 0.25) (layer "B.Cu") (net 8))
 (segment (start 110.0172 64.1683) (end 109.3547 64.8308) (width 0.25) (layer "B.Cu") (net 8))
 (segment (start 108.5022 64.8308) (end 78.524 94.809) (width 0.25) (layer "B.Cu") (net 8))
 (segment (start 108.3599 59.835) (end 109.2594 59.835) (width 0.25) (layer "B.Cu") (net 8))
 (segment (start 109.2594 59.835) (end 110.0172 60.5928) (width 0.25) (layer "B.Cu") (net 8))
 (segment (start 108.825 48.405) (end 108.825 49.5817) (width 0.25) (layer "B.Cu") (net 8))
 (segment (start 107.6026 50.4364) (end 107.6026 59.0777) (width 0.25) (layer "B.Cu") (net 8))
 (segment (start 125.2411 26.9661) (end 126.475 28.2) (width 0.25) (layer "B.Cu") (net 26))
 (segment (start 109.455 34.435) (end 116.9239 26.9661) (width 0.25) (layer "B.Cu") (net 26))
 (segment (start 92.2267 43.325) (end 101.1167 34.435) (width 0.25) (layer "B.Cu") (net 26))
 (segment (start 116.9239 26.9661) (end 125.2411 26.9661) (width 0.25) (layer "B.Cu") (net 26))
 (segment (start 101.1167 34.435) (end 109.455 34.435) (width 0.25) (layer "B.Cu") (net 26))
 (segment (start 91.05 43.325) (end 92.2267 43.325) (width 0.25) (layer "B.Cu") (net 26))
 (segment (start 109.14 147.025) (end 110.1189 146.0461) (width 0.25) (layer "F.Cu") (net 17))
 (segment (start 108.825 33.165) (end 108.825 34.3417) (width 0.25) (layer "F.Cu") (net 17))
 (segment (start 112.0323 37.1813) (end 112.0323 50.863) (width 0.25) (layer "F.Cu") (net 17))
 (segment (start 109.1927 34.3417) (end 112.0323 37.1813) (width 0.25) (layer "F.Cu") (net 17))
 (segment (start 108.825 34.3417) (end 109.1927 34.3417) (width 0.25) (layer "F.Cu") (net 17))
 (segment (start 110.1189 146.0461) (end 110.1189 59.3681) (width 0.25) (layer "F.Cu") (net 17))
 (via (at 110.1189 59.3681) (size 0.8) (drill 0.4) (layers "F.Cu" "B.Cu") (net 17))
 (via (at 112.0323 50.863) (size 0.8) (drill 0.4) (layers "F.Cu" "B.Cu") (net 17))
 (segment (start 110.1189 52.7764) (end 110.1189 59.3681) (width 0.25) (layer "B.Cu") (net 17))
 (segment (start 112.0323 50.863) (end 110.1189 52.7764) (width 0.25) (layer "B.Cu") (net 17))
 (segment (start 77.675 34.555) (end 74.005 38.225) (width 0.25) (layer "F.Cu") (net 4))
 (segment (start 77.675 29.275) (end 77.675 34.555) (width 0.25) (layer "F.Cu") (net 4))
 (segment (start 116.6608 146.8358) (end 116.85 147.025) (width 0.25) (layer "F.Cu") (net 20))
 (segment (start 116.6608 59.5898) (end 116.6608 146.8358) (width 0.25) (layer "F.Cu") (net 20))
 (segment (start 108.825 52.1217) (end 109.1927 52.1217) (width 0.25) (layer "F.Cu") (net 20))
 (segment (start 108.825 50.945) (end 108.825 52.1217) (width 0.25) (layer "F.Cu") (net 20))
 (segment (start 109.1927 52.1217) (end 116.6608 59.5898) (width 0.25) (layer "F.Cu") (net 20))
 (segment (start 87.8059 145.4531) (end 87.8059 93.0994) (width 0.25) (layer "F.Cu") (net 11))
 (segment (start 86.234 147.025) (end 87.8059 145.4531) (width 0.25) (layer "F.Cu") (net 11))
 (via (at 87.8059 93.0994) (size 0.8) (drill 0.4) (layers "F.Cu" "B.Cu") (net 11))
 (segment (start 108.825 72.4417) (end 108.4636 72.4417) (width 0.25) (layer "B.Cu") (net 11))
 (segment (start 108.825 71.265) (end 108.825 72.4417) (width 0.25) (layer "B.Cu") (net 11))
 (segment (start 108.4636 72.4417) (end 87.8059 93.0994) (width 0.25) (layer "B.Cu") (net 11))
 (segment (start 108.825 58.565) (end 108.825 59.7417) (width 0.25) (layer "F.Cu") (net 16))
 (segment (start 106.62 61.579) (end 108.4573 59.7417) (width 0.25) (layer "F.Cu") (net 16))
 (segment (start 106.62 147.025) (end 106.62 61.579) (width 0.25) (layer "F.Cu") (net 16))
 (segment (start 108.4573 59.7417) (end 108.825 59.7417) (width 0.25) (layer "F.Cu") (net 16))
 (segment (start 103.6179 62.1527) (end 103.6179 137.2511) (width 0.25) (layer "F.Cu") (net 14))
 (segment (start 103.6179 137.2511) (end 93.844 147.025) (width 0.25) (layer "F.Cu") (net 14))
 (via (at 103.6179 62.1527) (size 0.8) (drill 0.4) (layers "F.Cu" "B.Cu") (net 14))
 (segment (start 104.6656 61.105) (end 103.6179 62.1527) (width 0.25) (layer "B.Cu") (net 14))
 (segment (start 108.825 61.105) (end 104.6656 61.105) (width 0.25) (layer "B.Cu") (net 14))
 (segment (start 119.406 147.025) (end 117.3875 145.0065) (width 0.25) (layer "F.Cu") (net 21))
 (segment (start 117.3875 145.0065) (end 117.3875 74.7475) (width 0.25) (layer "F.Cu") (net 21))
 (via (at 117.3875 74.7475) (size 0.8) (drill 0.4) (layers "F.Cu" "B.Cu") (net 21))
 (segment (start 108.825 66.185) (end 110.0017 66.185) (width 0.25) (layer "B.Cu") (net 21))
 (segment (start 110.0017 66.185) (end 110.0017 67.3617) (width 0.25) (layer "B.Cu") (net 21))
 (segment (start 110.0017 67.3617) (end 117.3875 74.7475) (width 0.25) (layer "B.Cu") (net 21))
 (segment (start 108.825 53.485) (end 108.825 54.6617) (width 0.25) (layer "F.Cu") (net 19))
 (segment (start 114.299 59.768) (end 114.299 147.025) (width 0.25) (layer "F.Cu") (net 19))
 (segment (start 108.825 54.6617) (end 109.1927 54.6617) (width 0.25) (layer "F.Cu") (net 19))
 (segment (start 109.1927 54.6617) (end 114.299 59.768) (width 0.25) (layer "F.Cu") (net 19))
 (segment (start 108.825 57.2017) (end 109.1927 57.2017) (width 0.25) (layer "F.Cu") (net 18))
 (segment (start 109.1927 57.2017) (end 111.682 59.691) (width 0.25) (layer "F.Cu") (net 18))
 (segment (start 111.682 59.691) (end 111.682 147.025) (width 0.25) (layer "F.Cu") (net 18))
 (segment (start 108.825 56.025) (end 108.825 57.2017) (width 0.25) (layer "F.Cu") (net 18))
 (segment (start 102.7848 135.6142) (end 102.7848 76.8243) (width 0.25) (layer "F.Cu") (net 13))
 (segment (start 91.374 147.025) (end 102.7848 135.6142) (width 0.25) (layer "F.Cu") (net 13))
 (via (at 102.7848 76.8243) (size 0.8) (drill 0.4) (layers "F.Cu" "B.Cu") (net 13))
 (segment (start 102.7848 75.5742) (end 102.7848 76.8243) (width 0.25) (layer "B.Cu") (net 13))
 (segment (start 108.4573 69.9017) (end 102.7848 75.5742) (width 0.25) (layer "B.Cu") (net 13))
 (segment (start 108.825 68.725) (end 108.825 69.9017) (width 0.25) (layer "B.Cu") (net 13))
 (segment (start 108.825 69.9017) (end 108.4573 69.9017) (width 0.25) (layer "B.Cu") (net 13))
 (segment (start 91.05 57.3883) (end 90.6823 57.3883) (width 0.25) (layer "F.Cu") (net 5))
 (segment (start 91.05 58.565) (end 91.05 57.3883) (width 0.25) (layer "F.Cu") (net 5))
 (segment (start 90.6823 57.3883) (end 81.625 48.331) (width 0.25) (layer "F.Cu") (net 5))
 (segment (start 81.625 48.331) (end 81.625 38.225) (width 0.25) (layer "F.Cu") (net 5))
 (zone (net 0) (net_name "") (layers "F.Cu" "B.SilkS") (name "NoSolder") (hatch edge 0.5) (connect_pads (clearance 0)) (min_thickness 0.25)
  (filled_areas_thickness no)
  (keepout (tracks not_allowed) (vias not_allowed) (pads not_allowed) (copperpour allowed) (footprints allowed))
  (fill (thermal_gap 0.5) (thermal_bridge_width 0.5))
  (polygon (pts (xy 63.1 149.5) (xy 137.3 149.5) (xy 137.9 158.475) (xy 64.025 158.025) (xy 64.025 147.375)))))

